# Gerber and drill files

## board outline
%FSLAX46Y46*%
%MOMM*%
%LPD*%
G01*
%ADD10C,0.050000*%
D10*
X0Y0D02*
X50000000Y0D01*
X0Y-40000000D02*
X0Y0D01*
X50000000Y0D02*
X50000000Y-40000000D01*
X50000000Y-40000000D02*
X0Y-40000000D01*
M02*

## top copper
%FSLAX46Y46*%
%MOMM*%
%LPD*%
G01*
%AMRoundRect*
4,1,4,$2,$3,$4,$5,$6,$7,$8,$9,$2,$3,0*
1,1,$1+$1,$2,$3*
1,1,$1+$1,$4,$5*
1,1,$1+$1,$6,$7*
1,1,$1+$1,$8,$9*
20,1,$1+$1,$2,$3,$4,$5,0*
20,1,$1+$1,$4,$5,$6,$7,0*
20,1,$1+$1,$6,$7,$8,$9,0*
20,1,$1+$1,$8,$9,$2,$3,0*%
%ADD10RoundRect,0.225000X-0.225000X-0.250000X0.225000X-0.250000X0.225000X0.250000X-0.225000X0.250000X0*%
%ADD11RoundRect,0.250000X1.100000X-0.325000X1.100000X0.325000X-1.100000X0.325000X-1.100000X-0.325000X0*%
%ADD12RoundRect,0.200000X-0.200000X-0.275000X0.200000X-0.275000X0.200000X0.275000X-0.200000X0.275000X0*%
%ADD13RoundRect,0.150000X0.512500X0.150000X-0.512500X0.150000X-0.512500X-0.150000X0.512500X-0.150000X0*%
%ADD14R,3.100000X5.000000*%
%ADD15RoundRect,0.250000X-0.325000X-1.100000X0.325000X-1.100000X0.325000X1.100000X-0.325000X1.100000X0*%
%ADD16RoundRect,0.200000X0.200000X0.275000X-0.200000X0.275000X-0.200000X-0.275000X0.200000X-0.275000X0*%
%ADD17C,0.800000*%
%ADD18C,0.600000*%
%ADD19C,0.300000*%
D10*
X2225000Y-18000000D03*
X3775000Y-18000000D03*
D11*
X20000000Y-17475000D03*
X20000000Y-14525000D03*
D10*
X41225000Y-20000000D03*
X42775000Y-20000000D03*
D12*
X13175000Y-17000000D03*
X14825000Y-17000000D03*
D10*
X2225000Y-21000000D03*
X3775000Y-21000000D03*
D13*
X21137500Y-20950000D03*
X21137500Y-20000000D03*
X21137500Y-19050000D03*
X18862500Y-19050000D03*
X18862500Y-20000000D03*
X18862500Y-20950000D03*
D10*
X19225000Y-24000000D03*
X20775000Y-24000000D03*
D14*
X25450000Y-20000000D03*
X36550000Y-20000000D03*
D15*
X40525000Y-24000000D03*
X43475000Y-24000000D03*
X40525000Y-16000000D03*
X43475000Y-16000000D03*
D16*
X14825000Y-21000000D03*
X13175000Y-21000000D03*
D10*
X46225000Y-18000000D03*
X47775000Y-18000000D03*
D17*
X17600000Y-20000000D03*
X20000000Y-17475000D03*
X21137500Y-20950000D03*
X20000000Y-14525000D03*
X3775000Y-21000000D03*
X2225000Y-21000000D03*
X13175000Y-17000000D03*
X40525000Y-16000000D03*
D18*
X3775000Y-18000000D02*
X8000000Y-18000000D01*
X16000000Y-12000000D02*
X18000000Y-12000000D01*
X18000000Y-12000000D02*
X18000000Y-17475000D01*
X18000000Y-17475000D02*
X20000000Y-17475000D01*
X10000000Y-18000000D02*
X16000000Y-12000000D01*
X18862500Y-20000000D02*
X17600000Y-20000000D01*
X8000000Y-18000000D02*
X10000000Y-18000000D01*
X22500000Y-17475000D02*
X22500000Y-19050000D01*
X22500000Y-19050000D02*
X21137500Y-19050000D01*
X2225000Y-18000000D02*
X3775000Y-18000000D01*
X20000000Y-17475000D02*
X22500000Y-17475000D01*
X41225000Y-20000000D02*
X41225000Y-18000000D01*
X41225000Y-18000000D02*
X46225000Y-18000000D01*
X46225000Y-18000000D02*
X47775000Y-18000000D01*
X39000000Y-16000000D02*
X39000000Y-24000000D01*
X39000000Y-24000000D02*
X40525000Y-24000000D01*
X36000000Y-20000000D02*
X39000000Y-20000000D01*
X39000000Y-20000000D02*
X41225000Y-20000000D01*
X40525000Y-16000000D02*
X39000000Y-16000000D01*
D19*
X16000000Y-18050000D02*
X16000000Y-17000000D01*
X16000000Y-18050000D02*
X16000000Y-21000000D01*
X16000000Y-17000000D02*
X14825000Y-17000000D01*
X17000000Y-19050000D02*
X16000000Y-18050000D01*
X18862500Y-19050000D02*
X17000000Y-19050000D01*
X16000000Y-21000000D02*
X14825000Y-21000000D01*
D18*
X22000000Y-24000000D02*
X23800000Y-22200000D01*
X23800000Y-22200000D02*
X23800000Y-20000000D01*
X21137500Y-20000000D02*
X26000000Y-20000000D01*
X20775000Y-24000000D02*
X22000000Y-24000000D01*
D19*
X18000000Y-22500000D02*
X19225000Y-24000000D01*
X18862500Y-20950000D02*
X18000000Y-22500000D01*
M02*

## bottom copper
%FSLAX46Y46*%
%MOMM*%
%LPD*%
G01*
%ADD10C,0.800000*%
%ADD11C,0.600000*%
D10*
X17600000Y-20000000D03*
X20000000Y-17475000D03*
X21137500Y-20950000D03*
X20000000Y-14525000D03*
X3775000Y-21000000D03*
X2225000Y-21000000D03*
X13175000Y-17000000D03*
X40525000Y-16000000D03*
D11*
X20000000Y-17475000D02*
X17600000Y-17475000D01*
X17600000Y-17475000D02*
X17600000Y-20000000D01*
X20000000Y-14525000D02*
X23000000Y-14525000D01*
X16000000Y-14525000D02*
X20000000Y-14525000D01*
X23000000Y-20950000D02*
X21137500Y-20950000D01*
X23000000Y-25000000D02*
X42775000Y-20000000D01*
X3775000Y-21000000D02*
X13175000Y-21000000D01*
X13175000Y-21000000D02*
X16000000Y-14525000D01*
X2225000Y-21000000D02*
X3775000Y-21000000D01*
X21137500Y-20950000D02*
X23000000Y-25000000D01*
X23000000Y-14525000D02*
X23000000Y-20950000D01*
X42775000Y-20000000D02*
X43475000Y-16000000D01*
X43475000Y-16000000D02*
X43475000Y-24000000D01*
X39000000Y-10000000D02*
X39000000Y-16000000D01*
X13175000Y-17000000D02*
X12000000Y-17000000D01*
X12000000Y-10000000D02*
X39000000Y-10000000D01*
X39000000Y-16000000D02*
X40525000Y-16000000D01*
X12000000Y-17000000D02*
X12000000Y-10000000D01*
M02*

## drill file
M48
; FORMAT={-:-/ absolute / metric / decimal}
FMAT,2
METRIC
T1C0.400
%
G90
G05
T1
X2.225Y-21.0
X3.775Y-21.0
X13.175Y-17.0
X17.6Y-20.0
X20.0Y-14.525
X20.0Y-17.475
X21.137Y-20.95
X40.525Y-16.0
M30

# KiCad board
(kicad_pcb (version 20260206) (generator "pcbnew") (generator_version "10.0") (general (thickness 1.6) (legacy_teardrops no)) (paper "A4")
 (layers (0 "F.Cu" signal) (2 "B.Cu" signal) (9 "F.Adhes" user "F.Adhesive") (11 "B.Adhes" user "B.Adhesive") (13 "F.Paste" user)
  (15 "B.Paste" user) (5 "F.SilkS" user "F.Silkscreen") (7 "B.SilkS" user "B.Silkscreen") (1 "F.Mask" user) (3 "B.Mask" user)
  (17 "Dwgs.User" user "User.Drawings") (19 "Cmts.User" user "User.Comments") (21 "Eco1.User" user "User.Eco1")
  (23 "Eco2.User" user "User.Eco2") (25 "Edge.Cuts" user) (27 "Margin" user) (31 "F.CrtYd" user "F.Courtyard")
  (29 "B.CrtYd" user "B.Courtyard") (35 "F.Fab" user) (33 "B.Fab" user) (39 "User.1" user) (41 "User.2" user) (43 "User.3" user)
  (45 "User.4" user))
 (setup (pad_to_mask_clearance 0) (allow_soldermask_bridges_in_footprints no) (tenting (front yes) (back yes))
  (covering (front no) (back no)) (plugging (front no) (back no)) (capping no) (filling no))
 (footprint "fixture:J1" (layer "F.Cu") (at 3 18)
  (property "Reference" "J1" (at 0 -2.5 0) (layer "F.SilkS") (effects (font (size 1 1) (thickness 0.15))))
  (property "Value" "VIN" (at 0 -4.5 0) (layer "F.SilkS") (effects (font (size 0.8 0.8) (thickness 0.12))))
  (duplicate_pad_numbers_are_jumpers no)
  (pad "1" smd roundrect (at -0.775 0) (size 0.9 0.95) (layers "F.Cu" "F.Mask" "F.Paste") (roundrect_rratio 0.25) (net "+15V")
   (thermal_bridge_angle 45))
  (pad "2" smd roundrect (at 0.775 0) (size 0.9 0.95) (layers "F.Cu" "F.Mask" "F.Paste") (roundrect_rratio 0.25) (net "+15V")
   (thermal_bridge_angle 45)))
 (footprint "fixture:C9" (layer "F.Cu") (at 20 16 90)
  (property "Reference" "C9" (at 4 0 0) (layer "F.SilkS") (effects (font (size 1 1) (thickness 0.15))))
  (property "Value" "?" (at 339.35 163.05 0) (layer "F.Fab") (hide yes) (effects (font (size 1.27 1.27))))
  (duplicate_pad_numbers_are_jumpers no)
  (pad "1" smd roundrect (at -1.475 0 90) (size 1.15 2.7) (layers "F.Cu" "F.Mask" "F.Paste") (roundrect_rratio 0.217391) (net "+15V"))
  (pad "2" smd roundrect (at 1.475 0 90) (size 1.15 2.7) (layers "F.Cu" "F.Mask" "F.Paste") (roundrect_rratio 0.217391) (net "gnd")))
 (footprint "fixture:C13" (layer "F.Cu") (at 42 20)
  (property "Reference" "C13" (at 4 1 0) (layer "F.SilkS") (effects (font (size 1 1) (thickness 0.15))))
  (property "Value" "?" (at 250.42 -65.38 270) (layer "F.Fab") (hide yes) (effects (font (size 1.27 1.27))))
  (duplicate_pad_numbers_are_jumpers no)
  (pad "1" smd roundrect (at -0.775 0) (size 0.9 0.95) (layers "F.Cu" "F.Mask" "F.Paste") (roundrect_rratio 0.25) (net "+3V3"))
  (pad "2" smd roundrect (at 0.775 0) (size 0.9 0.95) (layers "F.Cu" "F.Mask" "F.Paste") (roundrect_rratio 0.25) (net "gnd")))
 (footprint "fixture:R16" (layer "F.Cu") (at 14 17)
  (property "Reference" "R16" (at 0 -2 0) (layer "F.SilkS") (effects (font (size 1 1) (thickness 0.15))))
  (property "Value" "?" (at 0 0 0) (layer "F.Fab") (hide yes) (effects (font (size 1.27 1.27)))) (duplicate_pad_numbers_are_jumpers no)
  (pad "1" smd roundrect (at -0.825 0) (size 0.8 0.95) (layers "F.Cu" "F.Mask" "F.Paste") (roundrect_rratio 0.25) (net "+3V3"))
  (pad "2" smd roundrect (at 0.825 0) (size 0.8 0.95) (layers "F.Cu" "F.Mask" "F.Paste") (roundrect_rratio 0.25) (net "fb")))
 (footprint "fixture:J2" (layer "F.Cu") (at 3 21)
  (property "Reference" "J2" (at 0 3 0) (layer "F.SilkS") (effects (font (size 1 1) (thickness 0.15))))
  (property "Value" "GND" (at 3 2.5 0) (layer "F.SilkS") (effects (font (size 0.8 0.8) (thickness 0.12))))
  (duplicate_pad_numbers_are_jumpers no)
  (pad "1" smd roundrect (at -0.775 0) (size 0.9 0.95) (layers "F.Cu" "F.Mask" "F.Paste") (roundrect_rratio 0.25) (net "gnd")
   (thermal_bridge_angle 45))
  (pad "2" smd roundrect (at 0.775 0) (size 0.9 0.95) (layers "F.Cu" "F.Mask" "F.Paste") (roundrect_rratio 0.25) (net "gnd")
   (thermal_bridge_angle 45)))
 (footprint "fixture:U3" (layer "F.Cu") (at 20 20 180)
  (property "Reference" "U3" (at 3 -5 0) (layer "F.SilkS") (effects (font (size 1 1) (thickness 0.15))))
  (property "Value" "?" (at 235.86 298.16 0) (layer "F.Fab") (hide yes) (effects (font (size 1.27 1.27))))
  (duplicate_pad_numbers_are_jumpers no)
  (pad "1" smd roundrect (at -1.1375 -0.95 180) (size 1.325 0.6) (layers "F.Cu" "F.Mask" "F.Paste") (roundrect_rratio 0.25) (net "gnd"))
  (pad "2" smd roundrect (at -1.1375 0 180) (size 1.325 0.6) (layers "F.Cu" "F.Mask" "F.Paste") (roundrect_rratio 0.25) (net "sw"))
  (pad "3" smd roundrect (at -1.1375 0.95 180) (size 1.325 0.6) (layers "F.Cu" "F.Mask" "F.Paste") (roundrect_rratio 0.25) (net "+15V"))
  (pad "4" smd roundrect (at 1.1375 0.95 180) (size 1.325 0.6) (layers "F.Cu" "F.Mask" "F.Paste") (roundrect_rratio 0.25) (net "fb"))
  (pad "5" smd roundrect (at 1.1375 0 180) (size 1.325 0.6) (layers "F.Cu" "F.Mask" "F.Paste") (roundrect_rratio 0.25) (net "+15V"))
  (pad "6" smd roundrect (at 1.1375 -0.95 180) (size 1.325 0.6) (layers "F.Cu" "F.Mask" "F.Paste") (roundrect_rratio 0.25) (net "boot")))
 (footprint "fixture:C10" (layer "F.Cu") (at 20 24)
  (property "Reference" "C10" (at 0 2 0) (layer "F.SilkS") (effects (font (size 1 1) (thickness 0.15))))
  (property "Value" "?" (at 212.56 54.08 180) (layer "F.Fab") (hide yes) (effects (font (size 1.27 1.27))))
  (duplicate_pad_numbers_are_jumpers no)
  (pad "1" smd roundrect (at -0.775 0) (size 0.9 0.95) (layers "F.Cu" "F.Mask" "F.Paste") (roundrect_rratio 0.25) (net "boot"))
  (pad "2" smd roundrect (at 0.775 0) (size 0.9 0.95) (layers "F.Cu" "F.Mask" "F.Paste") (roundrect_rratio 0.25) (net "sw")))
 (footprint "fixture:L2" (layer "F.Cu") (at 31 20)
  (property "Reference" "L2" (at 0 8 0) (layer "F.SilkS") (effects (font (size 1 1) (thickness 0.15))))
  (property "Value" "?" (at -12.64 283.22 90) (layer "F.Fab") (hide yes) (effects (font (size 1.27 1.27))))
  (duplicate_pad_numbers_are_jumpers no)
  (pad "1" smd rect (at -5.55 0) (size 3.1 5) (layers "F.Cu" "F.Mask" "F.Paste") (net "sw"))
  (pad "2" smd rect (at 5.55 0) (size 3.1 5) (layers "F.Cu" "F.Mask" "F.Paste") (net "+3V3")))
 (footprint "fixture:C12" (layer "F.Cu") (at 42 24)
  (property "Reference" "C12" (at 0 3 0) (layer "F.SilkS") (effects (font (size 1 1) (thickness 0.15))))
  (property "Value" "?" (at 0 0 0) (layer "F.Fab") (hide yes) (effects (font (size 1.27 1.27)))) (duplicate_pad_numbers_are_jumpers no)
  (pad "1" smd roundrect (at -1.475 0) (size 1.15 2.7) (layers "F.Cu" "F.Mask" "F.Paste") (roundrect_rratio 0.217391) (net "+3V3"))
  (pad "2" smd roundrect (at 1.475 0) (size 1.15 2.7) (layers "F.Cu" "F.Mask" "F.Paste") (roundrect_rratio 0.217391) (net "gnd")))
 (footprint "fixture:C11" (layer "F.Cu") (at 42 16)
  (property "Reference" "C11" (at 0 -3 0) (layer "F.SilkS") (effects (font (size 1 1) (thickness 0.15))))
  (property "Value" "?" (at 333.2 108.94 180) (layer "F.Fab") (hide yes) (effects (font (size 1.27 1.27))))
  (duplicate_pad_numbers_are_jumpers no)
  (pad "1" smd roundrect (at -1.475 0) (size 1.15 2.7) (layers "F.Cu" "F.Mask" "F.Paste") (roundrect_rratio 0.217391) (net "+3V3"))
  (pad "2" smd roundrect (at 1.475 0) (size 1.15 2.7) (layers "F.Cu" "F.Mask" "F.Paste") (roundrect_rratio 0.217391) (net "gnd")))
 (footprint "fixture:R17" (layer "F.Cu") (at 14 21 180)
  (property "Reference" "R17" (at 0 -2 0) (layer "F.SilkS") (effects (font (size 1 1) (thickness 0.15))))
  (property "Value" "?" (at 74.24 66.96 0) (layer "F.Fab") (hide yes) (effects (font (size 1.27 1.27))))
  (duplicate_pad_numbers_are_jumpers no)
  (pad "1" smd roundrect (at -0.825 0 180) (size 0.8 0.95) (layers "F.Cu" "F.Mask" "F.Paste") (roundrect_rratio 0.25) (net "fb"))
  (pad "2" smd roundrect (at 0.825 0 180) (size 0.8 0.95) (layers "F.Cu" "F.Mask" "F.Paste") (roundrect_rratio 0.25) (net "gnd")))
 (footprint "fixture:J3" (layer "F.Cu") (at 47 18)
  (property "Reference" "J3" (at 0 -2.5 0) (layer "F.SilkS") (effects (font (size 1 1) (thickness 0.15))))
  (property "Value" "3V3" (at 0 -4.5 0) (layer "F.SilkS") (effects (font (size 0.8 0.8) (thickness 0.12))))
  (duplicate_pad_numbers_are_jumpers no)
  (pad "1" smd roundrect (at -0.775 0) (size 0.9 0.95) (layers "F.Cu" "F.Mask" "F.Paste") (roundrect_rratio 0.25) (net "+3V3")
   (thermal_bridge_angle 45))
  (pad "2" smd roundrect (at 0.775 0) (size 0.9 0.95) (layers "F.Cu" "F.Mask" "F.Paste") (roundrect_rratio 0.25) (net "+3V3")
   (thermal_bridge_angle 45)))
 (gr_line (start 0 0) (end 50 0) (stroke (width 0.05) (type default)) (layer "Edge.Cuts"))
 (gr_line (start 0 40) (end 0 0) (stroke (width 0.05) (type default)) (layer "Edge.Cuts"))
 (gr_line (start 50 0) (end 50 40) (stroke (width 0.05) (type default)) (layer "Edge.Cuts"))
 (gr_line (start 50 40) (end 0 40) (stroke (width 0.05) (type default)) (layer "Edge.Cuts"))
 (segment (start 3.775 18) (end 8 18) (width 0.6) (layer "F.Cu") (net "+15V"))
 (segment (start 16 12) (end 18 12) (width 0.6) (layer "F.Cu") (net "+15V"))
 (segment (start 18 12) (end 18 17.475) (width 0.6) (layer "F.Cu") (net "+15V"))
 (segment (start 18 17.475) (end 20 17.475) (width 0.6) (layer "F.Cu") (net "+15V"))
 (segment (start 10 18) (end 16 12) (width 0.6) (layer "F.Cu") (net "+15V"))
 (segment (start 18.8625 20) (end 17.6 20) (width 0.6) (layer "F.Cu") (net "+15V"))
 (segment (start 8 18) (end 10 18) (width 0.6) (layer "F.Cu") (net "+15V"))
 (segment (start 22.5 17.475) (end 22.5 19.05) (width 0.6) (layer "F.Cu") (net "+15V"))
 (segment (start 22.5 19.05) (end 21.1375 19.05) (width 0.6) (layer "F.Cu") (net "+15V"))
 (segment (start 2.225 18) (end 3.775 18) (width 0.6) (layer "F.Cu") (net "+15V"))
 (segment (start 20 17.475) (end 22.5 17.475) (width 0.6) (layer "F.Cu") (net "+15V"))
 (via (at 17.6 20) (size 0.8) (drill 0.4) (layers "F.Cu" "B.Cu") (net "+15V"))
 (via (at 20 17.475) (size 0.8) (drill 0.4) (layers "F.Cu" "B.Cu") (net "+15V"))
 (segment (start 20 17.475) (end 17.6 17.475) (width 0.6) (layer "B.Cu") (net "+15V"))
 (segment (start 17.6 17.475) (end 17.6 20) (width 0.6) (layer "B.Cu") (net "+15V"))
 (via (at 21.1375 20.95) (size 0.8) (drill 0.4) (layers "F.Cu" "B.Cu") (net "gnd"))
 (via (at 20 14.525) (size 0.8) (drill 0.4) (layers "F.Cu" "B.Cu") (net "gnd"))
 (via (at 3.775 21) (size 0.8) (drill 0.4) (layers "F.Cu" "B.Cu") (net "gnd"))
 (via (at 2.225 21) (size 0.8) (drill 0.4) (layers "F.Cu" "B.Cu") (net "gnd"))
 (segment (start 20 14.525) (end 23 14.525) (width 0.6) (layer "B.Cu") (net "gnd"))
 (segment (start 16 14.525) (end 20 14.525) (width 0.6) (layer "B.Cu") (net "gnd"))
 (segment (start 23 20.95) (end 21.1375 20.95) (width 0.6) (layer "B.Cu") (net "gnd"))
 (segment (start 23 25) (end 42.775 20) (width 0.6) (layer "B.Cu") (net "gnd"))
 (segment (start 3.775 21) (end 13.175 21) (width 0.6) (layer "B.Cu") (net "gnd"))
 (segment (start 13.175 21) (end 16 14.525) (width 0.6) (layer "B.Cu") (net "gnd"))
 (segment (start 2.225 21) (end 3.775 21) (width 0.6) (layer "B.Cu") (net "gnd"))
 (segment (start 21.1375 20.95) (end 23 25) (width 0.6) (layer "B.Cu") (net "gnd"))
 (segment (start 23 14.525) (end 23 20.95) (width 0.6) (layer "B.Cu") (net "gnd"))
 (segment (start 42.775 20) (end 43.475 16) (width 0.6) (layer "B.Cu") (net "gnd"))
 (segment (start 43.475 16) (end 43.475 24) (width 0.6) (layer "B.Cu") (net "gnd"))
 (segment (start 41.225 20) (end 41.225 18) (width 0.6) (layer "F.Cu") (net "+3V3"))
 (segment (start 41.225 18) (end 46.225 18) (width 0.6) (layer "F.Cu") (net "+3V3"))
 (segment (start 46.225 18) (end 47.775 18) (width 0.6) (layer "F.Cu") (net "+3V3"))
 (segment (start 39 16) (end 39 24) (width 0.6) (layer "F.Cu") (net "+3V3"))
 (segment (start 39 24) (end 40.525 24) (width 0.6) (layer "F.Cu") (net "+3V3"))
 (segment (start 36 20) (end 39 20) (width 0.6) (layer "F.Cu") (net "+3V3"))
 (segment (start 39 20) (end 41.225 20) (width 0.6) (layer "F.Cu") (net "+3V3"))
 (segment (start 40.525 16) (end 39 16) (width 0.6) (layer "F.Cu") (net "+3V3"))
 (via (at 13.175 17) (size 0.8) (drill 0.4) (layers "F.Cu" "B.Cu") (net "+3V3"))
 (via (at 40.525 16) (size 0.8) (drill 0.4) (layers "F.Cu" "B.Cu") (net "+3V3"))
 (segment (start 39 10) (end 39 16) (width 0.6) (layer "B.Cu") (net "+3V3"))
 (segment (start 13.175 17) (end 12 17) (width 0.6) (layer "B.Cu") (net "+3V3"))
 (segment (start 12 10) (end 39 10) (width 0.6) (layer "B.Cu") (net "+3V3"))
 (segment (start 39 16) (end 40.525 16) (width 0.6) (layer "B.Cu") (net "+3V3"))
 (segment (start 12 17) (end 12 10) (width 0.6) (layer "B.Cu") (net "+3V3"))
 (segment (start 16 18.05) (end 16 17) (width 0.3) (layer "F.Cu") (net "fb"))
 (segment (start 16 18.05) (end 16 21) (width 0.3) (layer "F.Cu") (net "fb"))
 (segment (start 16 17) (end 14.825 17) (width 0.3) (layer "F.Cu") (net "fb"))
 (segment (start 17 19.05) (end 16 18.05) (width 0.3) (layer "F.Cu") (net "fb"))
 (segment (start 18.8625 19.05) (end 17 19.05) (width 0.3) (layer "F.Cu") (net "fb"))
 (segment (start 16 21) (end 14.825 21) (width 0.3) (layer "F.Cu") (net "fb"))
 (segment (start 22 24) (end 23.8 22.2) (width 0.6) (layer "F.Cu") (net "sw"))
 (segment (start 23.8 22.2) (end 23.8 20) (width 0.6) (layer "F.Cu") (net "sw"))
 (segment (start 21.1375 20) (end 26 20) (width 0.6) (layer "F.Cu") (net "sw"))
 (segment (start 20.775 24) (end 22 24) (width 0.6) (layer "F.Cu") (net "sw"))
 (segment (start 18 22.5) (end 19.225 24) (width 0.3) (layer "F.Cu") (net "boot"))
 (segment (start 18.8625 20.95) (end 18 22.5) (width 0.3) (layer "F.Cu") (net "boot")))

